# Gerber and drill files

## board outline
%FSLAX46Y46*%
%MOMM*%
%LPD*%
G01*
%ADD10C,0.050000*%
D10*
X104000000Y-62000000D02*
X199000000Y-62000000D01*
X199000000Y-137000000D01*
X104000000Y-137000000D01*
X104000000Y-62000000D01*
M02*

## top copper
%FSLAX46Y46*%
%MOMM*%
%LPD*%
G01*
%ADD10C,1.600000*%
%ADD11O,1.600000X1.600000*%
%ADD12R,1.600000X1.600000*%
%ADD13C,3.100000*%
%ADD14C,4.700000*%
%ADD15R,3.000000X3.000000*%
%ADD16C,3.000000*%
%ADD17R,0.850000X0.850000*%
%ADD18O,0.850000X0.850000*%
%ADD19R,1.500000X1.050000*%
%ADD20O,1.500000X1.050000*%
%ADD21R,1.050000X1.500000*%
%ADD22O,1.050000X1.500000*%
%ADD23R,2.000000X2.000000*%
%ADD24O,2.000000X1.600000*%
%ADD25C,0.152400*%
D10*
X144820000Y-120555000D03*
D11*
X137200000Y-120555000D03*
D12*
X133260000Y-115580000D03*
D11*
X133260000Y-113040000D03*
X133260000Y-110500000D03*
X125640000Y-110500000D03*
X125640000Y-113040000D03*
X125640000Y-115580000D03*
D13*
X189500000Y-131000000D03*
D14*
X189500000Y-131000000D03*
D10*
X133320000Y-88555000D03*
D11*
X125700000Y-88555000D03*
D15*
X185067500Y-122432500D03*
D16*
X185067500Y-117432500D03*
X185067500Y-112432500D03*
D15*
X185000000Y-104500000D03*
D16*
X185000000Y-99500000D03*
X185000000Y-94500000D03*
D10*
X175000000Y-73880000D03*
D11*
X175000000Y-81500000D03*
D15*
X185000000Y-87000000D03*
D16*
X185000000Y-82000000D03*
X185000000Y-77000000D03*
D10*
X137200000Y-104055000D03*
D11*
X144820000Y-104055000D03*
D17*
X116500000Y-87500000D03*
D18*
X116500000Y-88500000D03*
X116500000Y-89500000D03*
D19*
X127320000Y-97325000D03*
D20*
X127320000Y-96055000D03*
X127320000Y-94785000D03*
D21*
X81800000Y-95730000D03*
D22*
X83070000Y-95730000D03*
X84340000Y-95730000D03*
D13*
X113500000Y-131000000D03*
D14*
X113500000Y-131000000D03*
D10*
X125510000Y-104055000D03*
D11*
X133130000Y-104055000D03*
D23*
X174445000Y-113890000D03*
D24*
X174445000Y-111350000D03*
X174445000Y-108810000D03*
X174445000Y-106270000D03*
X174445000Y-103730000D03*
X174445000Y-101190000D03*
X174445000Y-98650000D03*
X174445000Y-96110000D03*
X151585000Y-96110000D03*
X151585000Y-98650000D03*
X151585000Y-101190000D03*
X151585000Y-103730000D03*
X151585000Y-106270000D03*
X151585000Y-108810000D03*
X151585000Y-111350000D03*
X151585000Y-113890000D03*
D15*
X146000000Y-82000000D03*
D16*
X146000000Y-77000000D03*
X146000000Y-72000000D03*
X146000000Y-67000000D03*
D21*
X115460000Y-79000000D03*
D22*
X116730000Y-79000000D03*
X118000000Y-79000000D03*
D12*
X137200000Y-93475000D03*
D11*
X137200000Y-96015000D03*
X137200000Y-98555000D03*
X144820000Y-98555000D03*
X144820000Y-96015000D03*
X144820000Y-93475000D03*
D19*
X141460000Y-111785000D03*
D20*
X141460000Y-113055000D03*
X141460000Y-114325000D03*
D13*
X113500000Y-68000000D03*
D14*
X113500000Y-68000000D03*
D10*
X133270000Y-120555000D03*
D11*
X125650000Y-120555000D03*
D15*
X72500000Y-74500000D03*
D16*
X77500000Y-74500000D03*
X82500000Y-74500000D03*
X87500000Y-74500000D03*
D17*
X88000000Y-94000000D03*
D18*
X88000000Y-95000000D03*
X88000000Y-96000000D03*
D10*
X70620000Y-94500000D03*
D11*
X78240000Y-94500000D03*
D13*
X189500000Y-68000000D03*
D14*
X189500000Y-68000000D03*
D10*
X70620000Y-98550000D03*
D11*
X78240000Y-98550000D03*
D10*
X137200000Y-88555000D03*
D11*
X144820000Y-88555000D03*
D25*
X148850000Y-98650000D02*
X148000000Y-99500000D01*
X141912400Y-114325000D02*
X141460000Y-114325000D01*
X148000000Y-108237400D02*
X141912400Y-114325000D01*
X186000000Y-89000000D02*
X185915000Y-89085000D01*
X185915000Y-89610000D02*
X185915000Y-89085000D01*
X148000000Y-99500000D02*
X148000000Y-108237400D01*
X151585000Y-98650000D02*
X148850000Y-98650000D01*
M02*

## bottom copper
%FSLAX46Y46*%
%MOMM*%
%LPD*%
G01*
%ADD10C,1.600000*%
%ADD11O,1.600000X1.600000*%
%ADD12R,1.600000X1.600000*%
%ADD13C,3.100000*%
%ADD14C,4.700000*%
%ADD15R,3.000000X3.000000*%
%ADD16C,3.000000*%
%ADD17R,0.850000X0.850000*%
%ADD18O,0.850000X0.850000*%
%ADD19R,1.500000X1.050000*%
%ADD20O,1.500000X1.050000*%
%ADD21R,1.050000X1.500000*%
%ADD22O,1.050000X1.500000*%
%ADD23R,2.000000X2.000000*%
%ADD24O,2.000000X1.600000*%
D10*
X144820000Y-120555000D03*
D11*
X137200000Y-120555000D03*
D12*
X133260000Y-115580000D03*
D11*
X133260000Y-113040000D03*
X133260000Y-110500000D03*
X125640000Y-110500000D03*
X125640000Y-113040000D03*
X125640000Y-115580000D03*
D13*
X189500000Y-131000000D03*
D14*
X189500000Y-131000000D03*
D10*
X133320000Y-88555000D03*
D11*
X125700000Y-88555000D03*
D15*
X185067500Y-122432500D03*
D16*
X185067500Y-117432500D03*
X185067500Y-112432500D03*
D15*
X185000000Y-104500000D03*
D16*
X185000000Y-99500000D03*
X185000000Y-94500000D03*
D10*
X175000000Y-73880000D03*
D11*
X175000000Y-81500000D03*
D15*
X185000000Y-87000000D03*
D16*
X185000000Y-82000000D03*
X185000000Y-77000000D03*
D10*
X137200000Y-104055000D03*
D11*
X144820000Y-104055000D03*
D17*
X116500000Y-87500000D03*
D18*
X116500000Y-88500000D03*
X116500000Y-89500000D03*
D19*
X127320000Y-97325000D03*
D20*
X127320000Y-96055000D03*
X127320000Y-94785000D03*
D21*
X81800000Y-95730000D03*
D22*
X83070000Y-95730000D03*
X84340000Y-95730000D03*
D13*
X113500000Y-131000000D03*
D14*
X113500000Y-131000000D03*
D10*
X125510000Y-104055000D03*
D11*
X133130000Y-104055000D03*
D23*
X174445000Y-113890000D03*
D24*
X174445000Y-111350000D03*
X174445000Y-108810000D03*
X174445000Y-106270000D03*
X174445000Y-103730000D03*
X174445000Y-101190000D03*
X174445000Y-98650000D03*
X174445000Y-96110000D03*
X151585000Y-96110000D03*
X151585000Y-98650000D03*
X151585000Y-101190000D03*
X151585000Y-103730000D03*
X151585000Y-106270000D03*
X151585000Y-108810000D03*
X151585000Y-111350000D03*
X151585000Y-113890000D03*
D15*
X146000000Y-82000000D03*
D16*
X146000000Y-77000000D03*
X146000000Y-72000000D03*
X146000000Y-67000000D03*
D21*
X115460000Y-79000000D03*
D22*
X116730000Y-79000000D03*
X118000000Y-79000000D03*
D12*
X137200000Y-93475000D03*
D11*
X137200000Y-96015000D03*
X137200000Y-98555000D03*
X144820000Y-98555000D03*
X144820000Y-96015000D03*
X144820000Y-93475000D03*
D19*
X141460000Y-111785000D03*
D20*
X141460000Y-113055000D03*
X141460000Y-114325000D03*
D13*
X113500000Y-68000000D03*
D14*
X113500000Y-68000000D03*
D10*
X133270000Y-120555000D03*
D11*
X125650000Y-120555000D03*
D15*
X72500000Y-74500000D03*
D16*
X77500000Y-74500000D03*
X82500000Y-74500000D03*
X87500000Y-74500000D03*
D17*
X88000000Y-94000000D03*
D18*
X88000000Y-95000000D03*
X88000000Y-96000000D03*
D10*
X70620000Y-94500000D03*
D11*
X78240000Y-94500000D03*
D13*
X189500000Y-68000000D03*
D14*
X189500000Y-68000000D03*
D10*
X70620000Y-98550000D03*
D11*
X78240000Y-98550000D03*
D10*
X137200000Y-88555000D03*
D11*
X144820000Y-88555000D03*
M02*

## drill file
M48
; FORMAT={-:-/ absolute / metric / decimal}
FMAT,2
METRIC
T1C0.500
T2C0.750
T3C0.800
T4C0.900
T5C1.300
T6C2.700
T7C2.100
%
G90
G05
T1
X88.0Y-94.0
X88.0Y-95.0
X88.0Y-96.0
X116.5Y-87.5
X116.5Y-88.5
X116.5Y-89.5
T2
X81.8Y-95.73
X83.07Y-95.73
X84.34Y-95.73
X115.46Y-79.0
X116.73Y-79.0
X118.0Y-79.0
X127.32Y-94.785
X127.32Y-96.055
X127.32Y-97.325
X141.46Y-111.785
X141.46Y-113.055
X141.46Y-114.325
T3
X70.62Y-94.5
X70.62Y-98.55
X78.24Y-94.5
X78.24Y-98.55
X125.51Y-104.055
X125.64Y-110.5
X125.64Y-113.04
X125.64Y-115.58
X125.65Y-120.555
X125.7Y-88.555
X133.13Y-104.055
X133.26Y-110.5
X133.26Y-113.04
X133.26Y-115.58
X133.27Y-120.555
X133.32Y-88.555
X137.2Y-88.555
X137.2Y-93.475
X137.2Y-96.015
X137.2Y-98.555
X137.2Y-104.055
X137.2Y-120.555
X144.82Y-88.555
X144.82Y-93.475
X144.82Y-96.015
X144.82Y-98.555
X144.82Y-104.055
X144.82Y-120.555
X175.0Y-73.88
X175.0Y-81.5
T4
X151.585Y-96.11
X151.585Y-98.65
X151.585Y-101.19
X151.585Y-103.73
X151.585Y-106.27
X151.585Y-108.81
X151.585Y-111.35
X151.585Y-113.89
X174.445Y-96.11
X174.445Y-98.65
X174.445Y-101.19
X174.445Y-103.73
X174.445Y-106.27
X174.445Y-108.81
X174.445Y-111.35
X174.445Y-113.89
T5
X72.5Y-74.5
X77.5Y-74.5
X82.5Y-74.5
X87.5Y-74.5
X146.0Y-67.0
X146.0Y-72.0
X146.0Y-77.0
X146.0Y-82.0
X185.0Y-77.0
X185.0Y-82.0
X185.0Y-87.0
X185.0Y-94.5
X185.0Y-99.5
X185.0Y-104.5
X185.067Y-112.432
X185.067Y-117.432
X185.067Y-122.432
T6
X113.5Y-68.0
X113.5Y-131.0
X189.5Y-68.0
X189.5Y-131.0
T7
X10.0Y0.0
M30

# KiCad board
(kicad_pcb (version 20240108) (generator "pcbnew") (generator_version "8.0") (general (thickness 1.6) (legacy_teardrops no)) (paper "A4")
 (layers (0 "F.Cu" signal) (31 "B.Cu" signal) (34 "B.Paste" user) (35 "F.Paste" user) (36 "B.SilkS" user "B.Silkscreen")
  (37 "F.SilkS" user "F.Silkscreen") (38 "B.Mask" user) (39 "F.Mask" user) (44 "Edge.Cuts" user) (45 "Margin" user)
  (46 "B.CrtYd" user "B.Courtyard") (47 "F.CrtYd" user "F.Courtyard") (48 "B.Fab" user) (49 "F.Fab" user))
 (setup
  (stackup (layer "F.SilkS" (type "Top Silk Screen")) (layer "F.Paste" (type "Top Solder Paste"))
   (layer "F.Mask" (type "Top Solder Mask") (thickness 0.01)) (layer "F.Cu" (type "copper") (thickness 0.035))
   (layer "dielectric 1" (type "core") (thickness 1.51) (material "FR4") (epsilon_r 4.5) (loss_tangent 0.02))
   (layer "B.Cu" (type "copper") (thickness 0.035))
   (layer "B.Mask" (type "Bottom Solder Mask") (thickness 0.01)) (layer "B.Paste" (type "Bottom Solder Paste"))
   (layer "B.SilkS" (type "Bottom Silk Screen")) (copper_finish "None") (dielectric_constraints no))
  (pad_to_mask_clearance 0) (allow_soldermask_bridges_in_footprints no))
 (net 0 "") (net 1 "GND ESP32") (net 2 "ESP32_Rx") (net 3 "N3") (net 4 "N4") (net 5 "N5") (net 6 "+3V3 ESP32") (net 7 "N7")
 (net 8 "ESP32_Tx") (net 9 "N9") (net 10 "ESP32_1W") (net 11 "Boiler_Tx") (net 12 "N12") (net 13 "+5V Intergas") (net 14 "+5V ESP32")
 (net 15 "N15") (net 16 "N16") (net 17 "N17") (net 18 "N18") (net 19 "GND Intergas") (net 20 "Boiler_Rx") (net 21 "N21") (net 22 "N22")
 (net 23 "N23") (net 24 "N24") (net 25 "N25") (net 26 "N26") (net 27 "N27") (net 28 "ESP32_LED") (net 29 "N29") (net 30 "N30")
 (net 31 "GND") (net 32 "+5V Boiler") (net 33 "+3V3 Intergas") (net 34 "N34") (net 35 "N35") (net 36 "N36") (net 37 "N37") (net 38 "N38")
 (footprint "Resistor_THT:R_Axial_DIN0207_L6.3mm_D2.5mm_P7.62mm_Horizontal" (layer "F.Cu") (at 144.82 120.555 180)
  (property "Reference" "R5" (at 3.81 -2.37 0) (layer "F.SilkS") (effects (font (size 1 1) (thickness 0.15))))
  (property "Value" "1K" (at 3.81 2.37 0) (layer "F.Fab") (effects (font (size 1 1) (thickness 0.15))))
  (pad "1" thru_hole circle (at 0 0 180) (size 1.6 1.6) (drill 0.8) (layers "*.Cu" "*.Mask") (remove_unused_layers no) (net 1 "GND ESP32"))
  (pad "2" thru_hole oval (at 7.62 0 180) (size 1.6 1.6) (drill 0.8) (layers "*.Cu" "*.Mask") (remove_unused_layers no) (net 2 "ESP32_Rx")))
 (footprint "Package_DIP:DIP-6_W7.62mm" (layer "F.Cu") (at 133.26 115.58 180)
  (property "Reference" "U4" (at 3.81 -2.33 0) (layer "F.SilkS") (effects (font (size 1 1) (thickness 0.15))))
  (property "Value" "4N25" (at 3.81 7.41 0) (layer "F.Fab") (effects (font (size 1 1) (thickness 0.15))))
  (pad "1" thru_hole rect (at 0 0 180) (size 1.6 1.6) (drill 0.8) (layers "*.Cu" "*.Mask") (remove_unused_layers no) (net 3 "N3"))
  (pad "2" thru_hole oval (at 0 2.54 180) (size 1.6 1.6) (drill 0.8) (layers "*.Cu" "*.Mask") (remove_unused_layers no) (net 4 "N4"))
  (pad "3" thru_hole oval (at 0 5.08 180) (size 1.6 1.6) (drill 0.8) (layers "*.Cu" "*.Mask") (remove_unused_layers no) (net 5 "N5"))
  (pad "4" thru_hole oval (at 7.62 5.08 180) (size 1.6 1.6) (drill 0.8) (layers "*.Cu" "*.Mask") (remove_unused_layers no)
   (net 2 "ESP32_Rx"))
  (pad "5" thru_hole oval (at 7.62 2.54 180) (size 1.6 1.6) (drill 0.8) (layers "*.Cu" "*.Mask") (remove_unused_layers no)
   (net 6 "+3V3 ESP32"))
  (pad "6" thru_hole oval (at 7.62 0 180) (size 1.6 1.6) (drill 0.8) (layers "*.Cu" "*.Mask") (remove_unused_layers no) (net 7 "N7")))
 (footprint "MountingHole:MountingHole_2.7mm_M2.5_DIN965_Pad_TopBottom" (layer "F.Cu") (at 189.5 131)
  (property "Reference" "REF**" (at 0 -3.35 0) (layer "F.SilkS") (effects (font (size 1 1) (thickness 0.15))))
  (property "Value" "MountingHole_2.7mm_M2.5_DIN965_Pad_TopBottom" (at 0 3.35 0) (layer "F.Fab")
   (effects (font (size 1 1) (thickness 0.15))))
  (pad "1" thru_hole circle (at 0 0) (size 3.1 3.1) (drill 2.7) (layers "*.Cu" "*.Mask") (remove_unused_layers no))
  (pad "1" connect circle (at 0 0) (size 4.7 4.7) (layers "F.Cu" "F.Mask"))
  (pad "1" connect circle (at 0 0) (size 4.7 4.7) (layers "B.Cu" "B.Mask")))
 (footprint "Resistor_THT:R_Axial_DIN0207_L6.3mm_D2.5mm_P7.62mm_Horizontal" (layer "F.Cu") (at 133.32 88.555 180)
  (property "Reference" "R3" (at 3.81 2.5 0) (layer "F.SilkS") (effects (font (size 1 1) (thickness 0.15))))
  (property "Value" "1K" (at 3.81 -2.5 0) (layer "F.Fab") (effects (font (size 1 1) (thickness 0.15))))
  (pad "1" thru_hole circle (at 0 0 180) (size 1.6 1.6) (drill 0.8) (layers "*.Cu" "*.Mask") (remove_unused_layers no) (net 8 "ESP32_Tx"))
  (pad "2" thru_hole oval (at 7.62 0 180) (size 1.6 1.6) (drill 0.8) (layers "*.Cu" "*.Mask") (remove_unused_layers no) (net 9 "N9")))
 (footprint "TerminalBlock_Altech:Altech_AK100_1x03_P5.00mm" (layer "F.Cu") (at 185.0675 122.4325 90)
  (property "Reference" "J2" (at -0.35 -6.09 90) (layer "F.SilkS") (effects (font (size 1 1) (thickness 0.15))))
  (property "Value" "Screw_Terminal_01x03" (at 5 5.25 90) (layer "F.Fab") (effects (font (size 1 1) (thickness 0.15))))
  (pad "1" thru_hole rect (at 0 0 90) (size 3 3) (drill 1.3) (layers "*.Cu" "*.Mask") (remove_unused_layers no) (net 6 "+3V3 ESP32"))
  (pad "2" thru_hole circle (at 5 0 90) (size 3 3) (drill 1.3) (layers "*.Cu" "*.Mask") (remove_unused_layers no) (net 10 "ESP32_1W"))
  (pad "3" thru_hole circle (at 10 0 90) (size 3 3) (drill 1.3) (layers "*.Cu" "*.Mask") (remove_unused_layers no) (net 1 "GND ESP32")))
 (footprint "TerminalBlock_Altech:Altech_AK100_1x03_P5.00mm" (layer "F.Cu") (at 185 104.5 90)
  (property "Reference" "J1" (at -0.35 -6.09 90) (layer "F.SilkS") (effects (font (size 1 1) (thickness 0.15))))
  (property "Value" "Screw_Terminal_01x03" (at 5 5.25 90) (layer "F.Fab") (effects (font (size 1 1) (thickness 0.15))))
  (pad "1" thru_hole rect (at 0 0 90) (size 3 3) (drill 1.3) (layers "*.Cu" "*.Mask") (remove_unused_layers no) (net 6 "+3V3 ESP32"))
  (pad "2" thru_hole circle (at 5 0 90) (size 3 3) (drill 1.3) (layers "*.Cu" "*.Mask") (remove_unused_layers no) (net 10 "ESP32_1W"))
  (pad "3" thru_hole circle (at 10 0 90) (size 3 3) (drill 1.3) (layers "*.Cu" "*.Mask") (remove_unused_layers no) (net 1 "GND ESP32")))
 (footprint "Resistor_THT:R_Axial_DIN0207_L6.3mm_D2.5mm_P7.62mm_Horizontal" (layer "F.Cu") (at 175 73.88 -90)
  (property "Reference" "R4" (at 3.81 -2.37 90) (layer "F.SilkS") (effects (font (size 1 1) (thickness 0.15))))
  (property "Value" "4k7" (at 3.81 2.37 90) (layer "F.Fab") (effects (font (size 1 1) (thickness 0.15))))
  (pad "1" thru_hole circle (at 0 0 270) (size 1.6 1.6) (drill 0.8) (layers "*.Cu" "*.Mask") (remove_unused_layers no) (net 10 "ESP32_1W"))
  (pad "2" thru_hole oval (at 7.62 0 270) (size 1.6 1.6) (drill 0.8) (layers "*.Cu" "*.Mask") (remove_unused_layers no) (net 6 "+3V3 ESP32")))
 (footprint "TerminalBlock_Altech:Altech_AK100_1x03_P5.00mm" (layer "F.Cu") (at 185 87 90)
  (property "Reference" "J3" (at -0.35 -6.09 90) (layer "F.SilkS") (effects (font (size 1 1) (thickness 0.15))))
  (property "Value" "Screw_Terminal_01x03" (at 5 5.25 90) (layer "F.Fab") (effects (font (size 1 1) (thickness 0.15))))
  (pad "1" thru_hole rect (at 0 0 90) (size 3 3) (drill 1.3) (layers "*.Cu" "*.Mask") (remove_unused_layers no) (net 6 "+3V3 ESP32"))
  (pad "2" thru_hole circle (at 5 0 90) (size 3 3) (drill 1.3) (layers "*.Cu" "*.Mask") (remove_unused_layers no) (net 10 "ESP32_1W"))
  (pad "3" thru_hole circle (at 10 0 90) (size 3 3) (drill 1.3) (layers "*.Cu" "*.Mask") (remove_unused_layers no) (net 1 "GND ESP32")))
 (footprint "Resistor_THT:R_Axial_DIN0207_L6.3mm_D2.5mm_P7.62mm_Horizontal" (layer "F.Cu") (at 137.2 104.055)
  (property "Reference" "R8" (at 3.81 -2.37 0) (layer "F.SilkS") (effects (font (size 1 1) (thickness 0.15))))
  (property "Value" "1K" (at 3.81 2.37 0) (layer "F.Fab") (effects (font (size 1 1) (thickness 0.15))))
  (pad "1" thru_hole circle (at 0 0) (size 1.6 1.6) (drill 0.8) (layers "*.Cu" "*.Mask") (remove_unused_layers no) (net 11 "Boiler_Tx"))
  (pad "2" thru_hole oval (at 7.62 0) (size 1.6 1.6) (drill 0.8) (layers "*.Cu" "*.Mask") (remove_unused_layers no) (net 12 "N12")))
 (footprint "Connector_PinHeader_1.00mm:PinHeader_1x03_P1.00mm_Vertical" (layer "F.Cu") (at 116.5 87.5)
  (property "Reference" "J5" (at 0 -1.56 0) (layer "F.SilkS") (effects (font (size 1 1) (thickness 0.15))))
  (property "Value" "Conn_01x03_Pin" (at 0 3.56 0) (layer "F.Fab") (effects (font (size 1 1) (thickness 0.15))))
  (pad "1" thru_hole rect (at 0 0) (size 0.85 0.85) (drill 0.5) (layers "*.Cu" "*.Mask") (remove_unused_layers no) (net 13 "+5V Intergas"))
  (pad "2" thru_hole oval (at 0 1) (size 0.85 0.85) (drill 0.5) (layers "*.Cu" "*.Mask") (remove_unused_layers no) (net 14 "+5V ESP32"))
  (pad "3" thru_hole oval (at 0 2) (size 0.85 0.85) (drill 0.5) (layers "*.Cu" "*.Mask") (remove_unused_layers no) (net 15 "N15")))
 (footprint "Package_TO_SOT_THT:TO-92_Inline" (layer "F.Cu") (at 127.32 97.325 90)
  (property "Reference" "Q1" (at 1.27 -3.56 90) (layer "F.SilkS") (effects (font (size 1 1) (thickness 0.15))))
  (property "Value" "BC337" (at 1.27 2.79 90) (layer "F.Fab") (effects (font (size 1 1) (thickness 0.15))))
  (pad "1" thru_hole rect (at 0 0 90) (size 1.05 1.5) (drill 0.75) (layers "*.Cu" "*.Mask") (remove_unused_layers no) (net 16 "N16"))
  (pad "2" thru_hole oval (at 1.27 0 90) (size 1.05 1.5) (drill 0.75) (layers "*.Cu" "*.Mask") (remove_unused_layers no) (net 9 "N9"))
  (pad "3" thru_hole oval (at 2.54 0 90) (size 1.05 1.5) (drill 0.75) (layers "*.Cu" "*.Mask") (remove_unused_layers no) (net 1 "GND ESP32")))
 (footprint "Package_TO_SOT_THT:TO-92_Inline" (layer "F.Cu") (at 81.8 95.73)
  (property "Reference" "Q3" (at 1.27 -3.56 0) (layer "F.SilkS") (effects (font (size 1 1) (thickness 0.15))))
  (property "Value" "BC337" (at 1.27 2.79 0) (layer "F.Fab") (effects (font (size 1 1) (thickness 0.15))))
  (pad "1" thru_hole rect (at 0 0) (size 1.05 1.5) (drill 0.75) (layers "*.Cu" "*.Mask") (remove_unused_layers no) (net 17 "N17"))
  (pad "2" thru_hole oval (at 1.27 0) (size 1.05 1.5) (drill 0.75) (layers "*.Cu" "*.Mask") (remove_unused_layers no) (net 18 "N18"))
  (pad "3" thru_hole oval (at 2.54 0) (size 1.05 1.5) (drill 0.75) (layers "*.Cu" "*.Mask") (remove_unused_layers no) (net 1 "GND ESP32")))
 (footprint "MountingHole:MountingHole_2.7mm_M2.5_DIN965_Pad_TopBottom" (layer "F.Cu") (at 113.5 131)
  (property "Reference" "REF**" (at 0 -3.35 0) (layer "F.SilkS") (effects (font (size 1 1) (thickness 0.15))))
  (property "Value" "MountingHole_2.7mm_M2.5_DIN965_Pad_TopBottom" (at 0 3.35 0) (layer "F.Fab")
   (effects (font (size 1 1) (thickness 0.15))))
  (pad "1" thru_hole circle (at 0 0) (size 3.1 3.1) (drill 2.7) (layers "*.Cu" "*.Mask") (remove_unused_layers no))
  (pad "1" connect circle (at 0 0) (size 4.7 4.7) (layers "F.Cu" "F.Mask"))
  (pad "1" connect circle (at 0 0) (size 4.7 4.7) (layers "B.Cu" "B.Mask")))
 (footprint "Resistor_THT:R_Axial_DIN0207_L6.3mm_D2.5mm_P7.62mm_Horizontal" (layer "F.Cu") (at 125.51 104.055)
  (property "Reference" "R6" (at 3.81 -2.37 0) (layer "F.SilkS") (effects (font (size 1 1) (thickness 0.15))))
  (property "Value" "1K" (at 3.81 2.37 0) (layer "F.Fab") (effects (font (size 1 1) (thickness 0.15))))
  (pad "1" thru_hole circle (at 0 0) (size 1.6 1.6) (drill 0.8) (layers "*.Cu" "*.Mask") (remove_unused_layers no) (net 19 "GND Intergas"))
  (pad "2" thru_hole oval (at 7.62 0) (size 1.6 1.6) (drill 0.8) (layers "*.Cu" "*.Mask") (remove_unused_layers no) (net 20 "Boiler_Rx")))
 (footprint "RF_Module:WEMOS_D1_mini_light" (layer "F.Cu") (at 174.445 113.89 180)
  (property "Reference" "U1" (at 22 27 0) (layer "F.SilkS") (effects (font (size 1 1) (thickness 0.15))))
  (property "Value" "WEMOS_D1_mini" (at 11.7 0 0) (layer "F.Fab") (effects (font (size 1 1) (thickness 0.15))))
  (pad "1" thru_hole rect (at 0 0 180) (size 2 2) (drill 0.9) (layers "*.Cu" "*.Mask") (remove_unused_layers no) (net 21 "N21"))
  (pad "2" thru_hole oval (at 0 2.54 180) (size 2 1.6) (drill 0.9) (layers "*.Cu" "*.Mask") (remove_unused_layers no) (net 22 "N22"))
  (pad "3" thru_hole oval (at 0 5.08 180) (size 2 1.6) (drill 0.9) (layers "*.Cu" "*.Mask") (remove_unused_layers no) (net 10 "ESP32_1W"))
  (pad "4" thru_hole oval (at 0 7.62 180) (size 2 1.6) (drill 0.9) (layers "*.Cu" "*.Mask") (remove_unused_layers no) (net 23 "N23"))
  (pad "5" thru_hole oval (at 0 10.16 180) (size 2 1.6) (drill 0.9) (layers "*.Cu" "*.Mask") (remove_unused_layers no) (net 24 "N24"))
  (pad "6" thru_hole oval (at 0 12.7 180) (size 2 1.6) (drill 0.9) (layers "*.Cu" "*.Mask") (remove_unused_layers no) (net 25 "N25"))
  (pad "7" thru_hole oval (at 0 15.24 180) (size 2 1.6) (drill 0.9) (layers "*.Cu" "*.Mask") (remove_unused_layers no) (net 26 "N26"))
  (pad "8" thru_hole oval (at 0 17.78 180) (size 2 1.6) (drill 0.9) (layers "*.Cu" "*.Mask") (remove_unused_layers no) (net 6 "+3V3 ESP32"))
  (pad "9" thru_hole oval (at 22.86 17.78 180) (size 2 1.6) (drill 0.9) (layers "*.Cu" "*.Mask") (remove_unused_layers no)
   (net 14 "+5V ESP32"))
  (pad "10" thru_hole oval (at 22.86 15.24 180) (size 2 1.6) (drill 0.9) (layers "*.Cu" "*.Mask") (remove_unused_layers no)
   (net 1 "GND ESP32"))
  (pad "11" thru_hole oval (at 22.86 12.7 180) (size 2 1.6) (drill 0.9) (layers "*.Cu" "*.Mask") (remove_unused_layers no) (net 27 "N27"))
  (pad "12" thru_hole oval (at 22.86 10.16 180) (size 2 1.6) (drill 0.9) (layers "*.Cu" "*.Mask") (remove_unused_layers no)
   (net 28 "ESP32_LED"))
  (pad "13" thru_hole oval (at 22.86 7.62 180) (size 2 1.6) (drill 0.9) (layers "*.Cu" "*.Mask") (remove_unused_layers no) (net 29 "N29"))
  (pad "14" thru_hole oval (at 22.86 5.08 180) (size 2 1.6) (drill 0.9) (layers "*.Cu" "*.Mask") (remove_unused_layers no) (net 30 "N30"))
  (pad "15" thru_hole oval (at 22.86 2.54 180) (size 2 1.6) (drill 0.9) (layers "*.Cu" "*.Mask") (remove_unused_layers no)
   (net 2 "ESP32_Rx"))
  (pad "16" thru_hole oval (at 22.86 0 180) (size 2 1.6) (drill 0.9) (layers "*.Cu" "*.Mask") (remove_unused_layers no) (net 8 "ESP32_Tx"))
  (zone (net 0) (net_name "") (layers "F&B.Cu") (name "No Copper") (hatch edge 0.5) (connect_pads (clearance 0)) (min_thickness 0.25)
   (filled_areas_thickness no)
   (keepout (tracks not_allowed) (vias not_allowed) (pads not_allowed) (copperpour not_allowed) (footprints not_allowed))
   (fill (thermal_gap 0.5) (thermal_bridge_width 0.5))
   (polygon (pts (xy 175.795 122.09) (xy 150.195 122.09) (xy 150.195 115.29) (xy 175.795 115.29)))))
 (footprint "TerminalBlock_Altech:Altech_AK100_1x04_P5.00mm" (layer "F.Cu") (at 146 82 90)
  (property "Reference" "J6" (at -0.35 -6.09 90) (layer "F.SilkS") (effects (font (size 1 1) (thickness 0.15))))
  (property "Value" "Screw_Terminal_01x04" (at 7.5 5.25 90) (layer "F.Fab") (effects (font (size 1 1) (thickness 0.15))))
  (pad "1" thru_hole rect (at 0 0 90) (size 3 3) (drill 1.3) (layers "*.Cu" "*.Mask") (remove_unused_layers no) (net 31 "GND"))
  (pad "2" thru_hole circle (at 5 0 90) (size 3 3) (drill 1.3) (layers "*.Cu" "*.Mask") (remove_unused_layers no) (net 11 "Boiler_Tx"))
  (pad "3" thru_hole circle (at 10 0 90) (size 3 3) (drill 1.3) (layers "*.Cu" "*.Mask") (remove_unused_layers no) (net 20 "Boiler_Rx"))
  (pad "4" thru_hole circle (at 15 0 90) (size 3 3) (drill 1.3) (layers "*.Cu" "*.Mask") (remove_unused_layers no) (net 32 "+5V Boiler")))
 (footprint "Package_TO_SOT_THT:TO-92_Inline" (layer "F.Cu") (at 115.46 79)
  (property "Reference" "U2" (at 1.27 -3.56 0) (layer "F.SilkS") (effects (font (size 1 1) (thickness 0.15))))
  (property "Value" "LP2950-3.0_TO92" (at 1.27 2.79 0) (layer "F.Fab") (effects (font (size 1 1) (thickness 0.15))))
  (pad "1" thru_hole rect (at 0 0) (size 1.05 1.5) (drill 0.75) (layers "*.Cu" "*.Mask") (remove_unused_layers no) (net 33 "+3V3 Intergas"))
  (pad "2" thru_hole oval (at 1.27 0) (size 1.05 1.5) (drill 0.75) (layers "*.Cu" "*.Mask") (remove_unused_layers no)
   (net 19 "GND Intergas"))
  (pad "3" thru_hole oval (at 2.54 0) (size 1.05 1.5) (drill 0.75) (layers "*.Cu" "*.Mask") (remove_unused_layers no)
   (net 13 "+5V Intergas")))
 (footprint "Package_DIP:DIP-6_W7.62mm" (layer "F.Cu") (at 137.2 93.475)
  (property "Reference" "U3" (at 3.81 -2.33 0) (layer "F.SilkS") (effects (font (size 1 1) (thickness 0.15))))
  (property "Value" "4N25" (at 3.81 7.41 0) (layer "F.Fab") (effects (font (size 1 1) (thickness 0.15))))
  (pad "1" thru_hole rect (at 0 0) (size 1.6 1.6) (drill 0.8) (layers "*.Cu" "*.Mask") (remove_unused_layers no) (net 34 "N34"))
  (pad "2" thru_hole oval (at 0 2.54) (size 1.6 1.6) (drill 0.8) (layers "*.Cu" "*.Mask") (remove_unused_layers no) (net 16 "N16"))
  (pad "3" thru_hole oval (at 0 5.08) (size 1.6 1.6) (drill 0.8) (layers "*.Cu" "*.Mask") (remove_unused_layers no) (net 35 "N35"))
  (pad "4" thru_hole oval (at 7.62 5.08) (size 1.6 1.6) (drill 0.8) (layers "*.Cu" "*.Mask") (remove_unused_layers no) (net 20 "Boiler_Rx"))
  (pad "5" thru_hole oval (at 7.62 2.54) (size 1.6 1.6) (drill 0.8) (layers "*.Cu" "*.Mask") (remove_unused_layers no)
   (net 33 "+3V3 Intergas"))
  (pad "6" thru_hole oval (at 7.62 0) (size 1.6 1.6) (drill 0.8) (layers "*.Cu" "*.Mask") (remove_unused_layers no) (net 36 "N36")))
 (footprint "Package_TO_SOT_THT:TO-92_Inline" (layer "F.Cu") (at 141.46 111.785 -90)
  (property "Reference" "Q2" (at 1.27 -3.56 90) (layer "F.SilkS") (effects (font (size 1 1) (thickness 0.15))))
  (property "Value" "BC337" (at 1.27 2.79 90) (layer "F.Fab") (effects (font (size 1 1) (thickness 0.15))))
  (pad "1" thru_hole rect (at 0 0 270) (size 1.05 1.5) (drill 0.75) (layers "*.Cu" "*.Mask") (remove_unused_layers no) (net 4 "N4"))
  (pad "2" thru_hole oval (at 1.27 0 270) (size 1.05 1.5) (drill 0.75) (layers "*.Cu" "*.Mask") (remove_unused_layers no) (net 12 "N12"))
  (pad "3" thru_hole oval (at 2.54 0 270) (size 1.05 1.5) (drill 0.75) (layers "*.Cu" "*.Mask") (remove_unused_layers no)
   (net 19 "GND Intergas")))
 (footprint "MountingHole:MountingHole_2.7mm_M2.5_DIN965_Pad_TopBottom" (layer "F.Cu") (at 113.5 68)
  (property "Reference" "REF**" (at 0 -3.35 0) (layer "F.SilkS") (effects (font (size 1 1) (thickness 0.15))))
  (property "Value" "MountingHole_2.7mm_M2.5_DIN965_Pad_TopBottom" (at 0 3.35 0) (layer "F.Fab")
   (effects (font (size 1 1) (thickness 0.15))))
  (pad "1" thru_hole circle (at 0 0) (size 3.1 3.1) (drill 2.7) (layers "*.Cu" "*.Mask") (remove_unused_layers no))
  (pad "1" connect circle (at 0 0) (size 4.7 4.7) (layers "F.Cu" "F.Mask"))
  (pad "1" connect circle (at 0 0) (size 4.7 4.7) (layers "B.Cu" "B.Mask")))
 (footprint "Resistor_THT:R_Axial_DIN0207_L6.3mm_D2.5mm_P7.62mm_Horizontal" (layer "F.Cu") (at 133.27 120.555 180)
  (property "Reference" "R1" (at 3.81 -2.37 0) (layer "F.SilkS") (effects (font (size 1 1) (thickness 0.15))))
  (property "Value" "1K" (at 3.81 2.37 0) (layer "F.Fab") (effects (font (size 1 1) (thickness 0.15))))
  (pad "1" thru_hole circle (at 0 0 180) (size 1.6 1.6) (drill 0.8) (layers "*.Cu" "*.Mask") (remove_unused_layers no) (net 3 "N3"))
  (pad "2" thru_hole oval (at 7.62 0 180) (size 1.6 1.6) (drill 0.8) (layers "*.Cu" "*.Mask") (remove_unused_layers no)
   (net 33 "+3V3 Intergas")))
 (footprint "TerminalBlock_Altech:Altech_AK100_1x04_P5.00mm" (layer "F.Cu") (at 72.5 74.5)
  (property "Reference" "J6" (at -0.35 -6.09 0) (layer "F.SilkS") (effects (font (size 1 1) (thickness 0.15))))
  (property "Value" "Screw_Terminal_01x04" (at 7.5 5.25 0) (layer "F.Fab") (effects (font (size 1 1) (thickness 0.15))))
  (pad "1" thru_hole rect (at 0 0) (size 3 3) (drill 1.3) (layers "*.Cu" "*.Mask") (remove_unused_layers no) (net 13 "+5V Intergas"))
  (pad "2" thru_hole circle (at 5 0) (size 3 3) (drill 1.3) (layers "*.Cu" "*.Mask") (remove_unused_layers no) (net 20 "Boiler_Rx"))
  (pad "3" thru_hole circle (at 10 0) (size 3 3) (drill 1.3) (layers "*.Cu" "*.Mask") (remove_unused_layers no) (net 11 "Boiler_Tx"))
  (pad "4" thru_hole circle (at 15 0) (size 3 3) (drill 1.3) (layers "*.Cu" "*.Mask") (remove_unused_layers no) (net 19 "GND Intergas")))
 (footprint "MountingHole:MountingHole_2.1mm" (layer "F.Cu") (at 10 0)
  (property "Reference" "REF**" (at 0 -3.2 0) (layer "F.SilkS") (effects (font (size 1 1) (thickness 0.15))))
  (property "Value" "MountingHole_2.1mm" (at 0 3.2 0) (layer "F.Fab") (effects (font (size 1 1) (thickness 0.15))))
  (pad "" np_thru_hole circle (at 0 0) (size 2.1 2.1) (drill 2.1) (layers "*.Cu" "*.Mask")))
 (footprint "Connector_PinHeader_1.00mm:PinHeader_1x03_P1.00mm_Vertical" (layer "F.Cu") (at 88 94)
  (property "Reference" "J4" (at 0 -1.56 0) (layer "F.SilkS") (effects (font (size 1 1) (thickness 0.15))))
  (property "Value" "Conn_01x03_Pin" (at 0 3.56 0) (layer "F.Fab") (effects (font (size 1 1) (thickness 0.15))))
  (pad "1" thru_hole rect (at 0 0) (size 0.85 0.85) (drill 0.5) (layers "*.Cu" "*.Mask") (remove_unused_layers no) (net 19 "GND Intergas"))
  (pad "2" thru_hole oval (at 0 1) (size 0.85 0.85) (drill 0.5) (layers "*.Cu" "*.Mask") (remove_unused_layers no) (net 1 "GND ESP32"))
  (pad "3" thru_hole oval (at 0 2) (size 0.85 0.85) (drill 0.5) (layers "*.Cu" "*.Mask") (remove_unused_layers no) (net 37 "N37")))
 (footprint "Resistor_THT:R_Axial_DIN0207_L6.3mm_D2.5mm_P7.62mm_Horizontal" (layer "F.Cu") (at 70.62 94.5)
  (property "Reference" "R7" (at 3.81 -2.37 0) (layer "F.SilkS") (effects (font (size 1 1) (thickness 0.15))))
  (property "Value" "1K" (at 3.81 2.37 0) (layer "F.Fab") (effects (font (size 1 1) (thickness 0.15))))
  (pad "1" thru_hole circle (at 0 0) (size 1.6 1.6) (drill 0.8) (layers "*.Cu" "*.Mask") (remove_unused_layers no) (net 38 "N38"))
  (pad "2" thru_hole oval (at 7.62 0) (size 1.6 1.6) (drill 0.8) (layers "*.Cu" "*.Mask") (remove_unused_layers no) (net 14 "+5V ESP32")))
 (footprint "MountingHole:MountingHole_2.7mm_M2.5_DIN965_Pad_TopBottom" (layer "F.Cu") (at 189.5 68)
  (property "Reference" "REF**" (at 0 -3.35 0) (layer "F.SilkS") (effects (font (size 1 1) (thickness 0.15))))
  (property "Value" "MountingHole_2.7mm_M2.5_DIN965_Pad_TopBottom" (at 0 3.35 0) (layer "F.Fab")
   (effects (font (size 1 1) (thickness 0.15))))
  (pad "1" thru_hole circle (at 0 0) (size 3.1 3.1) (drill 2.7) (layers "*.Cu" "*.Mask") (remove_unused_layers no))
  (pad "1" connect circle (at 0 0) (size 4.7 4.7) (layers "F.Cu" "F.Mask"))
  (pad "1" connect circle (at 0 0) (size 4.7 4.7) (layers "B.Cu" "B.Mask")))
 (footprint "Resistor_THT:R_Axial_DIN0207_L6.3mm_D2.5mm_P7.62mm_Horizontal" (layer "F.Cu") (at 70.62 98.55)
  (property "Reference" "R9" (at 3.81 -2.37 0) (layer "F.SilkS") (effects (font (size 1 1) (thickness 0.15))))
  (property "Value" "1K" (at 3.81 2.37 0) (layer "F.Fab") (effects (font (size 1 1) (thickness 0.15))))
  (pad "1" thru_hole circle (at 0 0) (size 1.6 1.6) (drill 0.8) (layers "*.Cu" "*.Mask") (remove_unused_layers no) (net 18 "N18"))
  (pad "2" thru_hole oval (at 7.62 0) (size 1.6 1.6) (drill 0.8) (layers "*.Cu" "*.Mask") (remove_unused_layers no) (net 28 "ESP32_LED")))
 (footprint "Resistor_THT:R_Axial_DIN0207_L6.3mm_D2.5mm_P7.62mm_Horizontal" (layer "F.Cu") (at 137.2 88.555)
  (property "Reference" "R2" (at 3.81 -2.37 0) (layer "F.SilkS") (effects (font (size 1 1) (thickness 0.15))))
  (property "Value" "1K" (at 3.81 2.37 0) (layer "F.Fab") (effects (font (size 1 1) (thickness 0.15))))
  (pad "1" thru_hole circle (at 0 0) (size 1.6 1.6) (drill 0.8) (layers "*.Cu" "*.Mask") (remove_unused_layers no) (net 34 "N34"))
  (pad "2" thru_hole oval (at 7.62 0) (size 1.6 1.6) (drill 0.8) (layers "*.Cu" "*.Mask") (remove_unused_layers no) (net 6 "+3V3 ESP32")))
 (gr_rect (start 104 62) (end 199 137) (stroke (width 0.05) (type default)) (fill none) (layer "Edge.Cuts"))
 (segment (start 148.85 98.65) (end 148 99.5) (width 0.1524) (layer "F.Cu") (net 31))
 (segment (start 141.9124 114.325) (end 141.46 114.325) (width 0.1524) (layer "F.Cu") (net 31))
 (segment (start 148 108.2374) (end 141.9124 114.325) (width 0.1524) (layer "F.Cu") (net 31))
 (segment (start 186 89) (end 185.915 89.085) (width 0.1524) (layer "F.Cu") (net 31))
 (segment (start 185.915 89.61) (end 185.915 89.085) (width 0.1524) (layer "F.Cu") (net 31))
 (segment (start 148 99.5) (end 148 108.2374) (width 0.1524) (layer "F.Cu") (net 31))
 (segment (start 151.585 98.65) (end 148.85 98.65) (width 0.1524) (layer "F.Cu") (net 31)))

